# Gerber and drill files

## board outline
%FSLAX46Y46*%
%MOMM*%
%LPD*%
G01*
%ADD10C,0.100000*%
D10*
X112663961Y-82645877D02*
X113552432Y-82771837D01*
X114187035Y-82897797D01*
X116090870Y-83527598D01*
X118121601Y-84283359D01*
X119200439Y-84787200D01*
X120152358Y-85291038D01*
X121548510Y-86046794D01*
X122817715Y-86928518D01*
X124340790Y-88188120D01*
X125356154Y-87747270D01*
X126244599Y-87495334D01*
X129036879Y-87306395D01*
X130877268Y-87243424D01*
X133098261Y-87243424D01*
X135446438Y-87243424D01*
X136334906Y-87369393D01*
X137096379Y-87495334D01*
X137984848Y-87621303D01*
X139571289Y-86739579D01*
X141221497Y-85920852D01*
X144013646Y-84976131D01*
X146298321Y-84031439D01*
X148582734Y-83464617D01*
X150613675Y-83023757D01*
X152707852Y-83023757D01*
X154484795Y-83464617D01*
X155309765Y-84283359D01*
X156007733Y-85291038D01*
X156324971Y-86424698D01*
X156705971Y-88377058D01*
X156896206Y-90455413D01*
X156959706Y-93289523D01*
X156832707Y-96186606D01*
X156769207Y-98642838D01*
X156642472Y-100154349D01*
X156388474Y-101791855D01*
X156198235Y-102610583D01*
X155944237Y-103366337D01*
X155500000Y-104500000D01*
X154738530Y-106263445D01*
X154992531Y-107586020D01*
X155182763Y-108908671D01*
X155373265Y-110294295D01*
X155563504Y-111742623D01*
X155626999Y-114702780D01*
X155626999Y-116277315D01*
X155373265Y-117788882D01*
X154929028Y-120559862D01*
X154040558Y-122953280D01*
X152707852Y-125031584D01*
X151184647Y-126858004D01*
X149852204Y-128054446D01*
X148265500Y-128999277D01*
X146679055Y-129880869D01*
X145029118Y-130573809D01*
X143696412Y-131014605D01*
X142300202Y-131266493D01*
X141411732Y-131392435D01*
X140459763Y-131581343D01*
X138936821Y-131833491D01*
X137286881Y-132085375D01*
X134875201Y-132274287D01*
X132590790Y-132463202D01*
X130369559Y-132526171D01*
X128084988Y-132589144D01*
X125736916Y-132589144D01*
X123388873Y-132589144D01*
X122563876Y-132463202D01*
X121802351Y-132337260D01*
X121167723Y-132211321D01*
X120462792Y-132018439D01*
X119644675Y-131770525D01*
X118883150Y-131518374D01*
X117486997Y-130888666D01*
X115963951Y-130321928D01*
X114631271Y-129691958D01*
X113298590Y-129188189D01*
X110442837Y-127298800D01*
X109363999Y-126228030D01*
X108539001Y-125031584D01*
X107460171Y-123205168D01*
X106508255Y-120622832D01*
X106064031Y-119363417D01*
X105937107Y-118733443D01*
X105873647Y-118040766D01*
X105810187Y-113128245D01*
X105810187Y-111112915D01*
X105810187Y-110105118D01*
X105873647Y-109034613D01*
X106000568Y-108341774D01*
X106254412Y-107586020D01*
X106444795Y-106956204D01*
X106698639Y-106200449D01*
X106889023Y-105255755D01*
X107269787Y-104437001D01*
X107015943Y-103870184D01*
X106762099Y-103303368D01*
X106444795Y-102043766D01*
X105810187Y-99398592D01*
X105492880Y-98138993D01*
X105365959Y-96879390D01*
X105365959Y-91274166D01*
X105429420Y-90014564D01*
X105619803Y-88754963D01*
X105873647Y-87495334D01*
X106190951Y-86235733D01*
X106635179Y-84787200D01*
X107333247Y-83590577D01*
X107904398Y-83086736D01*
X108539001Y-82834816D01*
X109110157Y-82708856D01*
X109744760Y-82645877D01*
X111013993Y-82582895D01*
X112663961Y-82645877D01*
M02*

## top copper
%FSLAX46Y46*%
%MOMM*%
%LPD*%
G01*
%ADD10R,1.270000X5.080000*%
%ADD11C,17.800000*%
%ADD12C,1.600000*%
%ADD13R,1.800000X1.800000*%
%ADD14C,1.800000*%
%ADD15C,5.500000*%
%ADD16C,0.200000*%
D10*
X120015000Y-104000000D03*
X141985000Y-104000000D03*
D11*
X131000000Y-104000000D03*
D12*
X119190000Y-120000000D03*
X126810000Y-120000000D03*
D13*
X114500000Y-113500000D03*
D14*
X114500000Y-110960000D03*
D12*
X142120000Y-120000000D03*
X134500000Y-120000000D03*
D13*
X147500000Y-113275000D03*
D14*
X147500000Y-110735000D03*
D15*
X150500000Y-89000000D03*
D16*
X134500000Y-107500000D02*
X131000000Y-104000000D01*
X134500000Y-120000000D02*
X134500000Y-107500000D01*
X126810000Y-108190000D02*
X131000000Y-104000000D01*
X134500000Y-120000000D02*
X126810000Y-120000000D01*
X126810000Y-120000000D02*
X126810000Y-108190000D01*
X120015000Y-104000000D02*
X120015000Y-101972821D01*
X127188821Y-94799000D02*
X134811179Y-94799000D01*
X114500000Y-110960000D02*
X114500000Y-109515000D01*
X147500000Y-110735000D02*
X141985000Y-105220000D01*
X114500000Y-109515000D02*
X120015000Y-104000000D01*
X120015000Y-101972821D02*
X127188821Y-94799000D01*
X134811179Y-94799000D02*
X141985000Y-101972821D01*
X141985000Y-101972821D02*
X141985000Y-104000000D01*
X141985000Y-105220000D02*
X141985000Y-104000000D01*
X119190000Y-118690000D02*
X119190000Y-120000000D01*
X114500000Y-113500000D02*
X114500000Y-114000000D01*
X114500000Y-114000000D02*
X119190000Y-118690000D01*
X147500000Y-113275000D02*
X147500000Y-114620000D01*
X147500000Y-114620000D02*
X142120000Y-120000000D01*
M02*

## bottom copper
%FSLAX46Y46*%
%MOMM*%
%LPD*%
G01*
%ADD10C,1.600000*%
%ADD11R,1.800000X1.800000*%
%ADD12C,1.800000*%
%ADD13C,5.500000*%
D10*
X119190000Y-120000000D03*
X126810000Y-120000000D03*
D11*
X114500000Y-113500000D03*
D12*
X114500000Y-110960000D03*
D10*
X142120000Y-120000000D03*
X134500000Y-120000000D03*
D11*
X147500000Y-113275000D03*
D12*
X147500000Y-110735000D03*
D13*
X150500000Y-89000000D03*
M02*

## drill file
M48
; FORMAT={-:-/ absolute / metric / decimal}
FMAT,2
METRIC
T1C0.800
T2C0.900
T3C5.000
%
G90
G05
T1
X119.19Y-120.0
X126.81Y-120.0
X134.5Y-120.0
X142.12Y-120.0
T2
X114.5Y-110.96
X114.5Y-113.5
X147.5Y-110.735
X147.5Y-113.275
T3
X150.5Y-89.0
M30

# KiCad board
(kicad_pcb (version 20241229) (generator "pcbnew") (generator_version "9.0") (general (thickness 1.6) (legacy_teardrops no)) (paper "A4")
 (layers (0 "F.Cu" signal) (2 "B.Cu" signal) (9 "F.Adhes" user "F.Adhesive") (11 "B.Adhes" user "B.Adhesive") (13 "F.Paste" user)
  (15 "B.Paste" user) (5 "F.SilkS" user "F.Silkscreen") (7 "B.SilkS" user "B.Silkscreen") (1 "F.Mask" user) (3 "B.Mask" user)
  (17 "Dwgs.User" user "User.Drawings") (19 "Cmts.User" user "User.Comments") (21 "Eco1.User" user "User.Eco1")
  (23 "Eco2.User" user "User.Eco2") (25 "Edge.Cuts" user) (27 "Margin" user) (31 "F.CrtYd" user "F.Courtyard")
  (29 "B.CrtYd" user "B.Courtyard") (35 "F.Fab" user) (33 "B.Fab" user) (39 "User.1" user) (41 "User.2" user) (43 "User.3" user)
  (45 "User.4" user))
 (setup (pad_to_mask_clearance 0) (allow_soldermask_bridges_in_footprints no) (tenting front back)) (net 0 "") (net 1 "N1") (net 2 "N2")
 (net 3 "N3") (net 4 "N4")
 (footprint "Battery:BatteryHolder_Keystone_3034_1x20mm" (layer "F.Cu") (at 131 104)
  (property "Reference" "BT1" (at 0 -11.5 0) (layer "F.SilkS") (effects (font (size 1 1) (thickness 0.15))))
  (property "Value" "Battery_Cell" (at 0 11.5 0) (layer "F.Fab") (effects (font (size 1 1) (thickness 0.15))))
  (pad "1" smd rect (at -10.985 0) (size 1.27 5.08) (layers "F.Cu" "F.Mask" "F.Paste") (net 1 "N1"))
  (pad "1" smd rect (at 10.985 0) (size 1.27 5.08) (layers "F.Cu" "F.Mask" "F.Paste") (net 1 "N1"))
  (pad "2" smd circle (at 0 0) (size 17.8 17.8) (layers "F.Cu" "F.Mask") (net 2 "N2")))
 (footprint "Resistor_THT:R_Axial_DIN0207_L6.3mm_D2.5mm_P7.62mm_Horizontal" (layer "F.Cu") (at 119.19 120)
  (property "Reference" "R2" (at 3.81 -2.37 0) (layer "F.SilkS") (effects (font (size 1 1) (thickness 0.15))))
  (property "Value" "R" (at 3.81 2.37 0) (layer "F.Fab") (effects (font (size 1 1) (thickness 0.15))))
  (pad "1" thru_hole circle (at 0 0) (size 1.6 1.6) (drill 0.8) (layers "*.Cu" "*.Mask") (remove_unused_layers no) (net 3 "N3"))
  (pad "2" thru_hole circle (at 7.62 0) (size 1.6 1.6) (drill 0.8) (layers "*.Cu" "*.Mask") (remove_unused_layers no) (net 2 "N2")))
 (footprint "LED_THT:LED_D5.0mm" (layer "F.Cu") (at 114.5 113.5 90)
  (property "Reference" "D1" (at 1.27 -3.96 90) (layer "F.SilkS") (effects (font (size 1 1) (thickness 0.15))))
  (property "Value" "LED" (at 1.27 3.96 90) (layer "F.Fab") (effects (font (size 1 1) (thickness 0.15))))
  (pad "1" thru_hole rect (at 0 0 90) (size 1.8 1.8) (drill 0.9) (layers "*.Cu" "*.Mask") (remove_unused_layers no) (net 3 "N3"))
  (pad "2" thru_hole circle (at 2.54 0 90) (size 1.8 1.8) (drill 0.9) (layers "*.Cu" "*.Mask") (remove_unused_layers no) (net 1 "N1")))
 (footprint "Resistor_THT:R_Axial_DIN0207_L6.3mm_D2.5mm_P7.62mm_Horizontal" (layer "F.Cu") (at 142.12 120 180)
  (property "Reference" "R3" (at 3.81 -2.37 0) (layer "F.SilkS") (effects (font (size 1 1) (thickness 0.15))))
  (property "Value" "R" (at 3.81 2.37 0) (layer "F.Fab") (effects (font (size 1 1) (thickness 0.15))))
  (pad "1" thru_hole circle (at 0 0 180) (size 1.6 1.6) (drill 0.8) (layers "*.Cu" "*.Mask") (remove_unused_layers no) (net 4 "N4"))
  (pad "2" thru_hole circle (at 7.62 0 180) (size 1.6 1.6) (drill 0.8) (layers "*.Cu" "*.Mask") (remove_unused_layers no) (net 2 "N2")))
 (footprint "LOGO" (layer "F.Cu") (at 114.5 93)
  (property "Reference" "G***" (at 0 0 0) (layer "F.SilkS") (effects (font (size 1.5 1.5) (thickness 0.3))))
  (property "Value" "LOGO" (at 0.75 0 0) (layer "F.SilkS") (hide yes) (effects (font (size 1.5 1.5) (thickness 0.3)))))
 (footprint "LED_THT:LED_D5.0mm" (layer "F.Cu") (at 147.5 113.275 90)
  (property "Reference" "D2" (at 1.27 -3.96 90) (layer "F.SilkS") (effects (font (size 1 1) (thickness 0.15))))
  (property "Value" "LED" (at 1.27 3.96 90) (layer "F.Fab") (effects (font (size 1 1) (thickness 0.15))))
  (pad "1" thru_hole rect (at 0 0 90) (size 1.8 1.8) (drill 0.9) (layers "*.Cu" "*.Mask") (remove_unused_layers no) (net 4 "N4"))
  (pad "2" thru_hole circle (at 2.54 0 90) (size 1.8 1.8) (drill 0.9) (layers "*.Cu" "*.Mask") (remove_unused_layers no) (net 1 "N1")))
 (gr_poly
  (pts (xy 112.663961 82.645877) (xy 113.552432 82.771837) (xy 114.187035 82.897797) (xy 116.09087 83.527598) (xy 118.121601 84.283359)
   (xy 119.200439 84.7872) (xy 120.152358 85.291038) (xy 121.54851 86.046794) (xy 122.817715 86.928518) (xy 124.34079 88.18812)
   (xy 125.356154 87.74727) (xy 126.244599 87.495334) (xy 129.036879 87.306395) (xy 130.877268 87.243424) (xy 133.098261 87.243424)
   (xy 135.446438 87.243424) (xy 136.334906 87.369393) (xy 137.096379 87.495334) (xy 137.984848 87.621303) (xy 139.571289 86.739579)
   (xy 141.221497 85.920852) (xy 144.013646 84.976131) (xy 146.298321 84.031439) (xy 148.582734 83.464617) (xy 150.613675 83.023757)
   (xy 152.707852 83.023757) (xy 154.484795 83.464617) (xy 155.309765 84.283359) (xy 156.007733 85.291038) (xy 156.324971 86.424698)
   (xy 156.705971 88.377058) (xy 156.896206 90.455413) (xy 156.959706 93.289523) (xy 156.832707 96.186606) (xy 156.769207 98.642838)
   (xy 156.642472 100.154349) (xy 156.388474 101.791855) (xy 156.198235 102.610583) (xy 155.944237 103.366337) (xy 155.5 104.5)
   (xy 154.73853 106.263445) (xy 154.992531 107.58602) (xy 155.182763 108.908671) (xy 155.373265 110.294295) (xy 155.563504 111.742623)
   (xy 155.626999 114.70278) (xy 155.626999 116.277315) (xy 155.373265 117.788882) (xy 154.929028 120.559862) (xy 154.040558 122.95328)
   (xy 152.707852 125.031584) (xy 151.184647 126.858004) (xy 149.852204 128.054446) (xy 148.2655 128.999277) (xy 146.679055 129.880869)
   (xy 145.029118 130.573809) (xy 143.696412 131.014605) (xy 142.300202 131.266493) (xy 141.411732 131.392435) (xy 140.459763 131.581343)
   (xy 138.936821 131.833491) (xy 137.286881 132.085375) (xy 134.875201 132.274287) (xy 132.59079 132.463202) (xy 130.369559 132.526171)
   (xy 128.084988 132.589144) (xy 125.736916 132.589144) (xy 123.388873 132.589144) (xy 122.563876 132.463202) (xy 121.802351 132.33726)
   (xy 121.167723 132.211321) (xy 120.462792 132.018439) (xy 119.644675 131.770525) (xy 118.88315 131.518374) (xy 117.486997 130.888666)
   (xy 115.963951 130.321928) (xy 114.631271 129.691958) (xy 113.29859 129.188189) (xy 110.442837 127.2988) (xy 109.363999 126.22803)
   (xy 108.539001 125.031584) (xy 107.460171 123.205168) (xy 106.508255 120.622832) (xy 106.064031 119.363417) (xy 105.937107 118.733443)
   (xy 105.873647 118.040766) (xy 105.810187 113.128245) (xy 105.810187 111.112915) (xy 105.810187 110.105118) (xy 105.873647 109.034613)
   (xy 106.000568 108.341774) (xy 106.254412 107.58602) (xy 106.444795 106.956204) (xy 106.698639 106.200449) (xy 106.889023 105.255755)
   (xy 107.269787 104.437001) (xy 107.015943 103.870184) (xy 106.762099 103.303368) (xy 106.444795 102.043766) (xy 105.810187 99.398592)
   (xy 105.49288 98.138993) (xy 105.365959 96.87939) (xy 105.365959 91.274166) (xy 105.42942 90.014564) (xy 105.619803 88.754963)
   (xy 105.873647 87.495334) (xy 106.190951 86.235733) (xy 106.635179 84.7872) (xy 107.333247 83.590577) (xy 107.904398 83.086736)
   (xy 108.539001 82.834816) (xy 109.110157 82.708856) (xy 109.74476 82.645877) (xy 111.013993 82.582895))
  (stroke (width 0.1) (type solid)) (fill no) (layer "Edge.Cuts"))
 (via (at 150.5 89) (size 5.5) (drill 5) (layers "F.Cu" "B.Cu") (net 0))
 (segment (start 134.5 107.5) (end 131 104) (width 0.2) (layer "F.Cu") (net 2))
 (segment (start 134.5 120) (end 134.5 107.5) (width 0.2) (layer "F.Cu") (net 2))
 (segment (start 126.81 108.19) (end 131 104) (width 0.2) (layer "F.Cu") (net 2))
 (segment (start 134.5 120) (end 126.81 120) (width 0.2) (layer "F.Cu") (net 2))
 (segment (start 126.81 120) (end 126.81 108.19) (width 0.2) (layer "F.Cu") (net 2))
 (segment (start 120.015 104) (end 120.015 101.972821) (width 0.2) (layer "F.Cu") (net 1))
 (segment (start 127.188821 94.799) (end 134.811179 94.799) (width 0.2) (layer "F.Cu") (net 1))
 (segment (start 114.5 110.96) (end 114.5 109.515) (width 0.2) (layer "F.Cu") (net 1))
 (segment (start 147.5 110.735) (end 141.985 105.22) (width 0.2) (layer "F.Cu") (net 1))
 (segment (start 114.5 109.515) (end 120.015 104) (width 0.2) (layer "F.Cu") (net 1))
 (segment (start 120.015 101.972821) (end 127.188821 94.799) (width 0.2) (layer "F.Cu") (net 1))
 (segment (start 134.811179 94.799) (end 141.985 101.972821) (width 0.2) (layer "F.Cu") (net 1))
 (segment (start 141.985 101.972821) (end 141.985 104) (width 0.2) (layer "F.Cu") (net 1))
 (segment (start 141.985 105.22) (end 141.985 104) (width 0.2) (layer "F.Cu") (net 1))
 (segment (start 119.19 118.69) (end 119.19 120) (width 0.2) (layer "F.Cu") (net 3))
 (segment (start 114.5 113.5) (end 114.5 114) (width 0.2) (layer "F.Cu") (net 3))
 (segment (start 114.5 114) (end 119.19 118.69) (width 0.2) (layer "F.Cu") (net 3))
 (segment (start 147.5 113.275) (end 147.5 114.62) (width 0.2) (layer "F.Cu") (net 4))
 (segment (start 147.5 114.62) (end 142.12 120) (width 0.2) (layer "F.Cu") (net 4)))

